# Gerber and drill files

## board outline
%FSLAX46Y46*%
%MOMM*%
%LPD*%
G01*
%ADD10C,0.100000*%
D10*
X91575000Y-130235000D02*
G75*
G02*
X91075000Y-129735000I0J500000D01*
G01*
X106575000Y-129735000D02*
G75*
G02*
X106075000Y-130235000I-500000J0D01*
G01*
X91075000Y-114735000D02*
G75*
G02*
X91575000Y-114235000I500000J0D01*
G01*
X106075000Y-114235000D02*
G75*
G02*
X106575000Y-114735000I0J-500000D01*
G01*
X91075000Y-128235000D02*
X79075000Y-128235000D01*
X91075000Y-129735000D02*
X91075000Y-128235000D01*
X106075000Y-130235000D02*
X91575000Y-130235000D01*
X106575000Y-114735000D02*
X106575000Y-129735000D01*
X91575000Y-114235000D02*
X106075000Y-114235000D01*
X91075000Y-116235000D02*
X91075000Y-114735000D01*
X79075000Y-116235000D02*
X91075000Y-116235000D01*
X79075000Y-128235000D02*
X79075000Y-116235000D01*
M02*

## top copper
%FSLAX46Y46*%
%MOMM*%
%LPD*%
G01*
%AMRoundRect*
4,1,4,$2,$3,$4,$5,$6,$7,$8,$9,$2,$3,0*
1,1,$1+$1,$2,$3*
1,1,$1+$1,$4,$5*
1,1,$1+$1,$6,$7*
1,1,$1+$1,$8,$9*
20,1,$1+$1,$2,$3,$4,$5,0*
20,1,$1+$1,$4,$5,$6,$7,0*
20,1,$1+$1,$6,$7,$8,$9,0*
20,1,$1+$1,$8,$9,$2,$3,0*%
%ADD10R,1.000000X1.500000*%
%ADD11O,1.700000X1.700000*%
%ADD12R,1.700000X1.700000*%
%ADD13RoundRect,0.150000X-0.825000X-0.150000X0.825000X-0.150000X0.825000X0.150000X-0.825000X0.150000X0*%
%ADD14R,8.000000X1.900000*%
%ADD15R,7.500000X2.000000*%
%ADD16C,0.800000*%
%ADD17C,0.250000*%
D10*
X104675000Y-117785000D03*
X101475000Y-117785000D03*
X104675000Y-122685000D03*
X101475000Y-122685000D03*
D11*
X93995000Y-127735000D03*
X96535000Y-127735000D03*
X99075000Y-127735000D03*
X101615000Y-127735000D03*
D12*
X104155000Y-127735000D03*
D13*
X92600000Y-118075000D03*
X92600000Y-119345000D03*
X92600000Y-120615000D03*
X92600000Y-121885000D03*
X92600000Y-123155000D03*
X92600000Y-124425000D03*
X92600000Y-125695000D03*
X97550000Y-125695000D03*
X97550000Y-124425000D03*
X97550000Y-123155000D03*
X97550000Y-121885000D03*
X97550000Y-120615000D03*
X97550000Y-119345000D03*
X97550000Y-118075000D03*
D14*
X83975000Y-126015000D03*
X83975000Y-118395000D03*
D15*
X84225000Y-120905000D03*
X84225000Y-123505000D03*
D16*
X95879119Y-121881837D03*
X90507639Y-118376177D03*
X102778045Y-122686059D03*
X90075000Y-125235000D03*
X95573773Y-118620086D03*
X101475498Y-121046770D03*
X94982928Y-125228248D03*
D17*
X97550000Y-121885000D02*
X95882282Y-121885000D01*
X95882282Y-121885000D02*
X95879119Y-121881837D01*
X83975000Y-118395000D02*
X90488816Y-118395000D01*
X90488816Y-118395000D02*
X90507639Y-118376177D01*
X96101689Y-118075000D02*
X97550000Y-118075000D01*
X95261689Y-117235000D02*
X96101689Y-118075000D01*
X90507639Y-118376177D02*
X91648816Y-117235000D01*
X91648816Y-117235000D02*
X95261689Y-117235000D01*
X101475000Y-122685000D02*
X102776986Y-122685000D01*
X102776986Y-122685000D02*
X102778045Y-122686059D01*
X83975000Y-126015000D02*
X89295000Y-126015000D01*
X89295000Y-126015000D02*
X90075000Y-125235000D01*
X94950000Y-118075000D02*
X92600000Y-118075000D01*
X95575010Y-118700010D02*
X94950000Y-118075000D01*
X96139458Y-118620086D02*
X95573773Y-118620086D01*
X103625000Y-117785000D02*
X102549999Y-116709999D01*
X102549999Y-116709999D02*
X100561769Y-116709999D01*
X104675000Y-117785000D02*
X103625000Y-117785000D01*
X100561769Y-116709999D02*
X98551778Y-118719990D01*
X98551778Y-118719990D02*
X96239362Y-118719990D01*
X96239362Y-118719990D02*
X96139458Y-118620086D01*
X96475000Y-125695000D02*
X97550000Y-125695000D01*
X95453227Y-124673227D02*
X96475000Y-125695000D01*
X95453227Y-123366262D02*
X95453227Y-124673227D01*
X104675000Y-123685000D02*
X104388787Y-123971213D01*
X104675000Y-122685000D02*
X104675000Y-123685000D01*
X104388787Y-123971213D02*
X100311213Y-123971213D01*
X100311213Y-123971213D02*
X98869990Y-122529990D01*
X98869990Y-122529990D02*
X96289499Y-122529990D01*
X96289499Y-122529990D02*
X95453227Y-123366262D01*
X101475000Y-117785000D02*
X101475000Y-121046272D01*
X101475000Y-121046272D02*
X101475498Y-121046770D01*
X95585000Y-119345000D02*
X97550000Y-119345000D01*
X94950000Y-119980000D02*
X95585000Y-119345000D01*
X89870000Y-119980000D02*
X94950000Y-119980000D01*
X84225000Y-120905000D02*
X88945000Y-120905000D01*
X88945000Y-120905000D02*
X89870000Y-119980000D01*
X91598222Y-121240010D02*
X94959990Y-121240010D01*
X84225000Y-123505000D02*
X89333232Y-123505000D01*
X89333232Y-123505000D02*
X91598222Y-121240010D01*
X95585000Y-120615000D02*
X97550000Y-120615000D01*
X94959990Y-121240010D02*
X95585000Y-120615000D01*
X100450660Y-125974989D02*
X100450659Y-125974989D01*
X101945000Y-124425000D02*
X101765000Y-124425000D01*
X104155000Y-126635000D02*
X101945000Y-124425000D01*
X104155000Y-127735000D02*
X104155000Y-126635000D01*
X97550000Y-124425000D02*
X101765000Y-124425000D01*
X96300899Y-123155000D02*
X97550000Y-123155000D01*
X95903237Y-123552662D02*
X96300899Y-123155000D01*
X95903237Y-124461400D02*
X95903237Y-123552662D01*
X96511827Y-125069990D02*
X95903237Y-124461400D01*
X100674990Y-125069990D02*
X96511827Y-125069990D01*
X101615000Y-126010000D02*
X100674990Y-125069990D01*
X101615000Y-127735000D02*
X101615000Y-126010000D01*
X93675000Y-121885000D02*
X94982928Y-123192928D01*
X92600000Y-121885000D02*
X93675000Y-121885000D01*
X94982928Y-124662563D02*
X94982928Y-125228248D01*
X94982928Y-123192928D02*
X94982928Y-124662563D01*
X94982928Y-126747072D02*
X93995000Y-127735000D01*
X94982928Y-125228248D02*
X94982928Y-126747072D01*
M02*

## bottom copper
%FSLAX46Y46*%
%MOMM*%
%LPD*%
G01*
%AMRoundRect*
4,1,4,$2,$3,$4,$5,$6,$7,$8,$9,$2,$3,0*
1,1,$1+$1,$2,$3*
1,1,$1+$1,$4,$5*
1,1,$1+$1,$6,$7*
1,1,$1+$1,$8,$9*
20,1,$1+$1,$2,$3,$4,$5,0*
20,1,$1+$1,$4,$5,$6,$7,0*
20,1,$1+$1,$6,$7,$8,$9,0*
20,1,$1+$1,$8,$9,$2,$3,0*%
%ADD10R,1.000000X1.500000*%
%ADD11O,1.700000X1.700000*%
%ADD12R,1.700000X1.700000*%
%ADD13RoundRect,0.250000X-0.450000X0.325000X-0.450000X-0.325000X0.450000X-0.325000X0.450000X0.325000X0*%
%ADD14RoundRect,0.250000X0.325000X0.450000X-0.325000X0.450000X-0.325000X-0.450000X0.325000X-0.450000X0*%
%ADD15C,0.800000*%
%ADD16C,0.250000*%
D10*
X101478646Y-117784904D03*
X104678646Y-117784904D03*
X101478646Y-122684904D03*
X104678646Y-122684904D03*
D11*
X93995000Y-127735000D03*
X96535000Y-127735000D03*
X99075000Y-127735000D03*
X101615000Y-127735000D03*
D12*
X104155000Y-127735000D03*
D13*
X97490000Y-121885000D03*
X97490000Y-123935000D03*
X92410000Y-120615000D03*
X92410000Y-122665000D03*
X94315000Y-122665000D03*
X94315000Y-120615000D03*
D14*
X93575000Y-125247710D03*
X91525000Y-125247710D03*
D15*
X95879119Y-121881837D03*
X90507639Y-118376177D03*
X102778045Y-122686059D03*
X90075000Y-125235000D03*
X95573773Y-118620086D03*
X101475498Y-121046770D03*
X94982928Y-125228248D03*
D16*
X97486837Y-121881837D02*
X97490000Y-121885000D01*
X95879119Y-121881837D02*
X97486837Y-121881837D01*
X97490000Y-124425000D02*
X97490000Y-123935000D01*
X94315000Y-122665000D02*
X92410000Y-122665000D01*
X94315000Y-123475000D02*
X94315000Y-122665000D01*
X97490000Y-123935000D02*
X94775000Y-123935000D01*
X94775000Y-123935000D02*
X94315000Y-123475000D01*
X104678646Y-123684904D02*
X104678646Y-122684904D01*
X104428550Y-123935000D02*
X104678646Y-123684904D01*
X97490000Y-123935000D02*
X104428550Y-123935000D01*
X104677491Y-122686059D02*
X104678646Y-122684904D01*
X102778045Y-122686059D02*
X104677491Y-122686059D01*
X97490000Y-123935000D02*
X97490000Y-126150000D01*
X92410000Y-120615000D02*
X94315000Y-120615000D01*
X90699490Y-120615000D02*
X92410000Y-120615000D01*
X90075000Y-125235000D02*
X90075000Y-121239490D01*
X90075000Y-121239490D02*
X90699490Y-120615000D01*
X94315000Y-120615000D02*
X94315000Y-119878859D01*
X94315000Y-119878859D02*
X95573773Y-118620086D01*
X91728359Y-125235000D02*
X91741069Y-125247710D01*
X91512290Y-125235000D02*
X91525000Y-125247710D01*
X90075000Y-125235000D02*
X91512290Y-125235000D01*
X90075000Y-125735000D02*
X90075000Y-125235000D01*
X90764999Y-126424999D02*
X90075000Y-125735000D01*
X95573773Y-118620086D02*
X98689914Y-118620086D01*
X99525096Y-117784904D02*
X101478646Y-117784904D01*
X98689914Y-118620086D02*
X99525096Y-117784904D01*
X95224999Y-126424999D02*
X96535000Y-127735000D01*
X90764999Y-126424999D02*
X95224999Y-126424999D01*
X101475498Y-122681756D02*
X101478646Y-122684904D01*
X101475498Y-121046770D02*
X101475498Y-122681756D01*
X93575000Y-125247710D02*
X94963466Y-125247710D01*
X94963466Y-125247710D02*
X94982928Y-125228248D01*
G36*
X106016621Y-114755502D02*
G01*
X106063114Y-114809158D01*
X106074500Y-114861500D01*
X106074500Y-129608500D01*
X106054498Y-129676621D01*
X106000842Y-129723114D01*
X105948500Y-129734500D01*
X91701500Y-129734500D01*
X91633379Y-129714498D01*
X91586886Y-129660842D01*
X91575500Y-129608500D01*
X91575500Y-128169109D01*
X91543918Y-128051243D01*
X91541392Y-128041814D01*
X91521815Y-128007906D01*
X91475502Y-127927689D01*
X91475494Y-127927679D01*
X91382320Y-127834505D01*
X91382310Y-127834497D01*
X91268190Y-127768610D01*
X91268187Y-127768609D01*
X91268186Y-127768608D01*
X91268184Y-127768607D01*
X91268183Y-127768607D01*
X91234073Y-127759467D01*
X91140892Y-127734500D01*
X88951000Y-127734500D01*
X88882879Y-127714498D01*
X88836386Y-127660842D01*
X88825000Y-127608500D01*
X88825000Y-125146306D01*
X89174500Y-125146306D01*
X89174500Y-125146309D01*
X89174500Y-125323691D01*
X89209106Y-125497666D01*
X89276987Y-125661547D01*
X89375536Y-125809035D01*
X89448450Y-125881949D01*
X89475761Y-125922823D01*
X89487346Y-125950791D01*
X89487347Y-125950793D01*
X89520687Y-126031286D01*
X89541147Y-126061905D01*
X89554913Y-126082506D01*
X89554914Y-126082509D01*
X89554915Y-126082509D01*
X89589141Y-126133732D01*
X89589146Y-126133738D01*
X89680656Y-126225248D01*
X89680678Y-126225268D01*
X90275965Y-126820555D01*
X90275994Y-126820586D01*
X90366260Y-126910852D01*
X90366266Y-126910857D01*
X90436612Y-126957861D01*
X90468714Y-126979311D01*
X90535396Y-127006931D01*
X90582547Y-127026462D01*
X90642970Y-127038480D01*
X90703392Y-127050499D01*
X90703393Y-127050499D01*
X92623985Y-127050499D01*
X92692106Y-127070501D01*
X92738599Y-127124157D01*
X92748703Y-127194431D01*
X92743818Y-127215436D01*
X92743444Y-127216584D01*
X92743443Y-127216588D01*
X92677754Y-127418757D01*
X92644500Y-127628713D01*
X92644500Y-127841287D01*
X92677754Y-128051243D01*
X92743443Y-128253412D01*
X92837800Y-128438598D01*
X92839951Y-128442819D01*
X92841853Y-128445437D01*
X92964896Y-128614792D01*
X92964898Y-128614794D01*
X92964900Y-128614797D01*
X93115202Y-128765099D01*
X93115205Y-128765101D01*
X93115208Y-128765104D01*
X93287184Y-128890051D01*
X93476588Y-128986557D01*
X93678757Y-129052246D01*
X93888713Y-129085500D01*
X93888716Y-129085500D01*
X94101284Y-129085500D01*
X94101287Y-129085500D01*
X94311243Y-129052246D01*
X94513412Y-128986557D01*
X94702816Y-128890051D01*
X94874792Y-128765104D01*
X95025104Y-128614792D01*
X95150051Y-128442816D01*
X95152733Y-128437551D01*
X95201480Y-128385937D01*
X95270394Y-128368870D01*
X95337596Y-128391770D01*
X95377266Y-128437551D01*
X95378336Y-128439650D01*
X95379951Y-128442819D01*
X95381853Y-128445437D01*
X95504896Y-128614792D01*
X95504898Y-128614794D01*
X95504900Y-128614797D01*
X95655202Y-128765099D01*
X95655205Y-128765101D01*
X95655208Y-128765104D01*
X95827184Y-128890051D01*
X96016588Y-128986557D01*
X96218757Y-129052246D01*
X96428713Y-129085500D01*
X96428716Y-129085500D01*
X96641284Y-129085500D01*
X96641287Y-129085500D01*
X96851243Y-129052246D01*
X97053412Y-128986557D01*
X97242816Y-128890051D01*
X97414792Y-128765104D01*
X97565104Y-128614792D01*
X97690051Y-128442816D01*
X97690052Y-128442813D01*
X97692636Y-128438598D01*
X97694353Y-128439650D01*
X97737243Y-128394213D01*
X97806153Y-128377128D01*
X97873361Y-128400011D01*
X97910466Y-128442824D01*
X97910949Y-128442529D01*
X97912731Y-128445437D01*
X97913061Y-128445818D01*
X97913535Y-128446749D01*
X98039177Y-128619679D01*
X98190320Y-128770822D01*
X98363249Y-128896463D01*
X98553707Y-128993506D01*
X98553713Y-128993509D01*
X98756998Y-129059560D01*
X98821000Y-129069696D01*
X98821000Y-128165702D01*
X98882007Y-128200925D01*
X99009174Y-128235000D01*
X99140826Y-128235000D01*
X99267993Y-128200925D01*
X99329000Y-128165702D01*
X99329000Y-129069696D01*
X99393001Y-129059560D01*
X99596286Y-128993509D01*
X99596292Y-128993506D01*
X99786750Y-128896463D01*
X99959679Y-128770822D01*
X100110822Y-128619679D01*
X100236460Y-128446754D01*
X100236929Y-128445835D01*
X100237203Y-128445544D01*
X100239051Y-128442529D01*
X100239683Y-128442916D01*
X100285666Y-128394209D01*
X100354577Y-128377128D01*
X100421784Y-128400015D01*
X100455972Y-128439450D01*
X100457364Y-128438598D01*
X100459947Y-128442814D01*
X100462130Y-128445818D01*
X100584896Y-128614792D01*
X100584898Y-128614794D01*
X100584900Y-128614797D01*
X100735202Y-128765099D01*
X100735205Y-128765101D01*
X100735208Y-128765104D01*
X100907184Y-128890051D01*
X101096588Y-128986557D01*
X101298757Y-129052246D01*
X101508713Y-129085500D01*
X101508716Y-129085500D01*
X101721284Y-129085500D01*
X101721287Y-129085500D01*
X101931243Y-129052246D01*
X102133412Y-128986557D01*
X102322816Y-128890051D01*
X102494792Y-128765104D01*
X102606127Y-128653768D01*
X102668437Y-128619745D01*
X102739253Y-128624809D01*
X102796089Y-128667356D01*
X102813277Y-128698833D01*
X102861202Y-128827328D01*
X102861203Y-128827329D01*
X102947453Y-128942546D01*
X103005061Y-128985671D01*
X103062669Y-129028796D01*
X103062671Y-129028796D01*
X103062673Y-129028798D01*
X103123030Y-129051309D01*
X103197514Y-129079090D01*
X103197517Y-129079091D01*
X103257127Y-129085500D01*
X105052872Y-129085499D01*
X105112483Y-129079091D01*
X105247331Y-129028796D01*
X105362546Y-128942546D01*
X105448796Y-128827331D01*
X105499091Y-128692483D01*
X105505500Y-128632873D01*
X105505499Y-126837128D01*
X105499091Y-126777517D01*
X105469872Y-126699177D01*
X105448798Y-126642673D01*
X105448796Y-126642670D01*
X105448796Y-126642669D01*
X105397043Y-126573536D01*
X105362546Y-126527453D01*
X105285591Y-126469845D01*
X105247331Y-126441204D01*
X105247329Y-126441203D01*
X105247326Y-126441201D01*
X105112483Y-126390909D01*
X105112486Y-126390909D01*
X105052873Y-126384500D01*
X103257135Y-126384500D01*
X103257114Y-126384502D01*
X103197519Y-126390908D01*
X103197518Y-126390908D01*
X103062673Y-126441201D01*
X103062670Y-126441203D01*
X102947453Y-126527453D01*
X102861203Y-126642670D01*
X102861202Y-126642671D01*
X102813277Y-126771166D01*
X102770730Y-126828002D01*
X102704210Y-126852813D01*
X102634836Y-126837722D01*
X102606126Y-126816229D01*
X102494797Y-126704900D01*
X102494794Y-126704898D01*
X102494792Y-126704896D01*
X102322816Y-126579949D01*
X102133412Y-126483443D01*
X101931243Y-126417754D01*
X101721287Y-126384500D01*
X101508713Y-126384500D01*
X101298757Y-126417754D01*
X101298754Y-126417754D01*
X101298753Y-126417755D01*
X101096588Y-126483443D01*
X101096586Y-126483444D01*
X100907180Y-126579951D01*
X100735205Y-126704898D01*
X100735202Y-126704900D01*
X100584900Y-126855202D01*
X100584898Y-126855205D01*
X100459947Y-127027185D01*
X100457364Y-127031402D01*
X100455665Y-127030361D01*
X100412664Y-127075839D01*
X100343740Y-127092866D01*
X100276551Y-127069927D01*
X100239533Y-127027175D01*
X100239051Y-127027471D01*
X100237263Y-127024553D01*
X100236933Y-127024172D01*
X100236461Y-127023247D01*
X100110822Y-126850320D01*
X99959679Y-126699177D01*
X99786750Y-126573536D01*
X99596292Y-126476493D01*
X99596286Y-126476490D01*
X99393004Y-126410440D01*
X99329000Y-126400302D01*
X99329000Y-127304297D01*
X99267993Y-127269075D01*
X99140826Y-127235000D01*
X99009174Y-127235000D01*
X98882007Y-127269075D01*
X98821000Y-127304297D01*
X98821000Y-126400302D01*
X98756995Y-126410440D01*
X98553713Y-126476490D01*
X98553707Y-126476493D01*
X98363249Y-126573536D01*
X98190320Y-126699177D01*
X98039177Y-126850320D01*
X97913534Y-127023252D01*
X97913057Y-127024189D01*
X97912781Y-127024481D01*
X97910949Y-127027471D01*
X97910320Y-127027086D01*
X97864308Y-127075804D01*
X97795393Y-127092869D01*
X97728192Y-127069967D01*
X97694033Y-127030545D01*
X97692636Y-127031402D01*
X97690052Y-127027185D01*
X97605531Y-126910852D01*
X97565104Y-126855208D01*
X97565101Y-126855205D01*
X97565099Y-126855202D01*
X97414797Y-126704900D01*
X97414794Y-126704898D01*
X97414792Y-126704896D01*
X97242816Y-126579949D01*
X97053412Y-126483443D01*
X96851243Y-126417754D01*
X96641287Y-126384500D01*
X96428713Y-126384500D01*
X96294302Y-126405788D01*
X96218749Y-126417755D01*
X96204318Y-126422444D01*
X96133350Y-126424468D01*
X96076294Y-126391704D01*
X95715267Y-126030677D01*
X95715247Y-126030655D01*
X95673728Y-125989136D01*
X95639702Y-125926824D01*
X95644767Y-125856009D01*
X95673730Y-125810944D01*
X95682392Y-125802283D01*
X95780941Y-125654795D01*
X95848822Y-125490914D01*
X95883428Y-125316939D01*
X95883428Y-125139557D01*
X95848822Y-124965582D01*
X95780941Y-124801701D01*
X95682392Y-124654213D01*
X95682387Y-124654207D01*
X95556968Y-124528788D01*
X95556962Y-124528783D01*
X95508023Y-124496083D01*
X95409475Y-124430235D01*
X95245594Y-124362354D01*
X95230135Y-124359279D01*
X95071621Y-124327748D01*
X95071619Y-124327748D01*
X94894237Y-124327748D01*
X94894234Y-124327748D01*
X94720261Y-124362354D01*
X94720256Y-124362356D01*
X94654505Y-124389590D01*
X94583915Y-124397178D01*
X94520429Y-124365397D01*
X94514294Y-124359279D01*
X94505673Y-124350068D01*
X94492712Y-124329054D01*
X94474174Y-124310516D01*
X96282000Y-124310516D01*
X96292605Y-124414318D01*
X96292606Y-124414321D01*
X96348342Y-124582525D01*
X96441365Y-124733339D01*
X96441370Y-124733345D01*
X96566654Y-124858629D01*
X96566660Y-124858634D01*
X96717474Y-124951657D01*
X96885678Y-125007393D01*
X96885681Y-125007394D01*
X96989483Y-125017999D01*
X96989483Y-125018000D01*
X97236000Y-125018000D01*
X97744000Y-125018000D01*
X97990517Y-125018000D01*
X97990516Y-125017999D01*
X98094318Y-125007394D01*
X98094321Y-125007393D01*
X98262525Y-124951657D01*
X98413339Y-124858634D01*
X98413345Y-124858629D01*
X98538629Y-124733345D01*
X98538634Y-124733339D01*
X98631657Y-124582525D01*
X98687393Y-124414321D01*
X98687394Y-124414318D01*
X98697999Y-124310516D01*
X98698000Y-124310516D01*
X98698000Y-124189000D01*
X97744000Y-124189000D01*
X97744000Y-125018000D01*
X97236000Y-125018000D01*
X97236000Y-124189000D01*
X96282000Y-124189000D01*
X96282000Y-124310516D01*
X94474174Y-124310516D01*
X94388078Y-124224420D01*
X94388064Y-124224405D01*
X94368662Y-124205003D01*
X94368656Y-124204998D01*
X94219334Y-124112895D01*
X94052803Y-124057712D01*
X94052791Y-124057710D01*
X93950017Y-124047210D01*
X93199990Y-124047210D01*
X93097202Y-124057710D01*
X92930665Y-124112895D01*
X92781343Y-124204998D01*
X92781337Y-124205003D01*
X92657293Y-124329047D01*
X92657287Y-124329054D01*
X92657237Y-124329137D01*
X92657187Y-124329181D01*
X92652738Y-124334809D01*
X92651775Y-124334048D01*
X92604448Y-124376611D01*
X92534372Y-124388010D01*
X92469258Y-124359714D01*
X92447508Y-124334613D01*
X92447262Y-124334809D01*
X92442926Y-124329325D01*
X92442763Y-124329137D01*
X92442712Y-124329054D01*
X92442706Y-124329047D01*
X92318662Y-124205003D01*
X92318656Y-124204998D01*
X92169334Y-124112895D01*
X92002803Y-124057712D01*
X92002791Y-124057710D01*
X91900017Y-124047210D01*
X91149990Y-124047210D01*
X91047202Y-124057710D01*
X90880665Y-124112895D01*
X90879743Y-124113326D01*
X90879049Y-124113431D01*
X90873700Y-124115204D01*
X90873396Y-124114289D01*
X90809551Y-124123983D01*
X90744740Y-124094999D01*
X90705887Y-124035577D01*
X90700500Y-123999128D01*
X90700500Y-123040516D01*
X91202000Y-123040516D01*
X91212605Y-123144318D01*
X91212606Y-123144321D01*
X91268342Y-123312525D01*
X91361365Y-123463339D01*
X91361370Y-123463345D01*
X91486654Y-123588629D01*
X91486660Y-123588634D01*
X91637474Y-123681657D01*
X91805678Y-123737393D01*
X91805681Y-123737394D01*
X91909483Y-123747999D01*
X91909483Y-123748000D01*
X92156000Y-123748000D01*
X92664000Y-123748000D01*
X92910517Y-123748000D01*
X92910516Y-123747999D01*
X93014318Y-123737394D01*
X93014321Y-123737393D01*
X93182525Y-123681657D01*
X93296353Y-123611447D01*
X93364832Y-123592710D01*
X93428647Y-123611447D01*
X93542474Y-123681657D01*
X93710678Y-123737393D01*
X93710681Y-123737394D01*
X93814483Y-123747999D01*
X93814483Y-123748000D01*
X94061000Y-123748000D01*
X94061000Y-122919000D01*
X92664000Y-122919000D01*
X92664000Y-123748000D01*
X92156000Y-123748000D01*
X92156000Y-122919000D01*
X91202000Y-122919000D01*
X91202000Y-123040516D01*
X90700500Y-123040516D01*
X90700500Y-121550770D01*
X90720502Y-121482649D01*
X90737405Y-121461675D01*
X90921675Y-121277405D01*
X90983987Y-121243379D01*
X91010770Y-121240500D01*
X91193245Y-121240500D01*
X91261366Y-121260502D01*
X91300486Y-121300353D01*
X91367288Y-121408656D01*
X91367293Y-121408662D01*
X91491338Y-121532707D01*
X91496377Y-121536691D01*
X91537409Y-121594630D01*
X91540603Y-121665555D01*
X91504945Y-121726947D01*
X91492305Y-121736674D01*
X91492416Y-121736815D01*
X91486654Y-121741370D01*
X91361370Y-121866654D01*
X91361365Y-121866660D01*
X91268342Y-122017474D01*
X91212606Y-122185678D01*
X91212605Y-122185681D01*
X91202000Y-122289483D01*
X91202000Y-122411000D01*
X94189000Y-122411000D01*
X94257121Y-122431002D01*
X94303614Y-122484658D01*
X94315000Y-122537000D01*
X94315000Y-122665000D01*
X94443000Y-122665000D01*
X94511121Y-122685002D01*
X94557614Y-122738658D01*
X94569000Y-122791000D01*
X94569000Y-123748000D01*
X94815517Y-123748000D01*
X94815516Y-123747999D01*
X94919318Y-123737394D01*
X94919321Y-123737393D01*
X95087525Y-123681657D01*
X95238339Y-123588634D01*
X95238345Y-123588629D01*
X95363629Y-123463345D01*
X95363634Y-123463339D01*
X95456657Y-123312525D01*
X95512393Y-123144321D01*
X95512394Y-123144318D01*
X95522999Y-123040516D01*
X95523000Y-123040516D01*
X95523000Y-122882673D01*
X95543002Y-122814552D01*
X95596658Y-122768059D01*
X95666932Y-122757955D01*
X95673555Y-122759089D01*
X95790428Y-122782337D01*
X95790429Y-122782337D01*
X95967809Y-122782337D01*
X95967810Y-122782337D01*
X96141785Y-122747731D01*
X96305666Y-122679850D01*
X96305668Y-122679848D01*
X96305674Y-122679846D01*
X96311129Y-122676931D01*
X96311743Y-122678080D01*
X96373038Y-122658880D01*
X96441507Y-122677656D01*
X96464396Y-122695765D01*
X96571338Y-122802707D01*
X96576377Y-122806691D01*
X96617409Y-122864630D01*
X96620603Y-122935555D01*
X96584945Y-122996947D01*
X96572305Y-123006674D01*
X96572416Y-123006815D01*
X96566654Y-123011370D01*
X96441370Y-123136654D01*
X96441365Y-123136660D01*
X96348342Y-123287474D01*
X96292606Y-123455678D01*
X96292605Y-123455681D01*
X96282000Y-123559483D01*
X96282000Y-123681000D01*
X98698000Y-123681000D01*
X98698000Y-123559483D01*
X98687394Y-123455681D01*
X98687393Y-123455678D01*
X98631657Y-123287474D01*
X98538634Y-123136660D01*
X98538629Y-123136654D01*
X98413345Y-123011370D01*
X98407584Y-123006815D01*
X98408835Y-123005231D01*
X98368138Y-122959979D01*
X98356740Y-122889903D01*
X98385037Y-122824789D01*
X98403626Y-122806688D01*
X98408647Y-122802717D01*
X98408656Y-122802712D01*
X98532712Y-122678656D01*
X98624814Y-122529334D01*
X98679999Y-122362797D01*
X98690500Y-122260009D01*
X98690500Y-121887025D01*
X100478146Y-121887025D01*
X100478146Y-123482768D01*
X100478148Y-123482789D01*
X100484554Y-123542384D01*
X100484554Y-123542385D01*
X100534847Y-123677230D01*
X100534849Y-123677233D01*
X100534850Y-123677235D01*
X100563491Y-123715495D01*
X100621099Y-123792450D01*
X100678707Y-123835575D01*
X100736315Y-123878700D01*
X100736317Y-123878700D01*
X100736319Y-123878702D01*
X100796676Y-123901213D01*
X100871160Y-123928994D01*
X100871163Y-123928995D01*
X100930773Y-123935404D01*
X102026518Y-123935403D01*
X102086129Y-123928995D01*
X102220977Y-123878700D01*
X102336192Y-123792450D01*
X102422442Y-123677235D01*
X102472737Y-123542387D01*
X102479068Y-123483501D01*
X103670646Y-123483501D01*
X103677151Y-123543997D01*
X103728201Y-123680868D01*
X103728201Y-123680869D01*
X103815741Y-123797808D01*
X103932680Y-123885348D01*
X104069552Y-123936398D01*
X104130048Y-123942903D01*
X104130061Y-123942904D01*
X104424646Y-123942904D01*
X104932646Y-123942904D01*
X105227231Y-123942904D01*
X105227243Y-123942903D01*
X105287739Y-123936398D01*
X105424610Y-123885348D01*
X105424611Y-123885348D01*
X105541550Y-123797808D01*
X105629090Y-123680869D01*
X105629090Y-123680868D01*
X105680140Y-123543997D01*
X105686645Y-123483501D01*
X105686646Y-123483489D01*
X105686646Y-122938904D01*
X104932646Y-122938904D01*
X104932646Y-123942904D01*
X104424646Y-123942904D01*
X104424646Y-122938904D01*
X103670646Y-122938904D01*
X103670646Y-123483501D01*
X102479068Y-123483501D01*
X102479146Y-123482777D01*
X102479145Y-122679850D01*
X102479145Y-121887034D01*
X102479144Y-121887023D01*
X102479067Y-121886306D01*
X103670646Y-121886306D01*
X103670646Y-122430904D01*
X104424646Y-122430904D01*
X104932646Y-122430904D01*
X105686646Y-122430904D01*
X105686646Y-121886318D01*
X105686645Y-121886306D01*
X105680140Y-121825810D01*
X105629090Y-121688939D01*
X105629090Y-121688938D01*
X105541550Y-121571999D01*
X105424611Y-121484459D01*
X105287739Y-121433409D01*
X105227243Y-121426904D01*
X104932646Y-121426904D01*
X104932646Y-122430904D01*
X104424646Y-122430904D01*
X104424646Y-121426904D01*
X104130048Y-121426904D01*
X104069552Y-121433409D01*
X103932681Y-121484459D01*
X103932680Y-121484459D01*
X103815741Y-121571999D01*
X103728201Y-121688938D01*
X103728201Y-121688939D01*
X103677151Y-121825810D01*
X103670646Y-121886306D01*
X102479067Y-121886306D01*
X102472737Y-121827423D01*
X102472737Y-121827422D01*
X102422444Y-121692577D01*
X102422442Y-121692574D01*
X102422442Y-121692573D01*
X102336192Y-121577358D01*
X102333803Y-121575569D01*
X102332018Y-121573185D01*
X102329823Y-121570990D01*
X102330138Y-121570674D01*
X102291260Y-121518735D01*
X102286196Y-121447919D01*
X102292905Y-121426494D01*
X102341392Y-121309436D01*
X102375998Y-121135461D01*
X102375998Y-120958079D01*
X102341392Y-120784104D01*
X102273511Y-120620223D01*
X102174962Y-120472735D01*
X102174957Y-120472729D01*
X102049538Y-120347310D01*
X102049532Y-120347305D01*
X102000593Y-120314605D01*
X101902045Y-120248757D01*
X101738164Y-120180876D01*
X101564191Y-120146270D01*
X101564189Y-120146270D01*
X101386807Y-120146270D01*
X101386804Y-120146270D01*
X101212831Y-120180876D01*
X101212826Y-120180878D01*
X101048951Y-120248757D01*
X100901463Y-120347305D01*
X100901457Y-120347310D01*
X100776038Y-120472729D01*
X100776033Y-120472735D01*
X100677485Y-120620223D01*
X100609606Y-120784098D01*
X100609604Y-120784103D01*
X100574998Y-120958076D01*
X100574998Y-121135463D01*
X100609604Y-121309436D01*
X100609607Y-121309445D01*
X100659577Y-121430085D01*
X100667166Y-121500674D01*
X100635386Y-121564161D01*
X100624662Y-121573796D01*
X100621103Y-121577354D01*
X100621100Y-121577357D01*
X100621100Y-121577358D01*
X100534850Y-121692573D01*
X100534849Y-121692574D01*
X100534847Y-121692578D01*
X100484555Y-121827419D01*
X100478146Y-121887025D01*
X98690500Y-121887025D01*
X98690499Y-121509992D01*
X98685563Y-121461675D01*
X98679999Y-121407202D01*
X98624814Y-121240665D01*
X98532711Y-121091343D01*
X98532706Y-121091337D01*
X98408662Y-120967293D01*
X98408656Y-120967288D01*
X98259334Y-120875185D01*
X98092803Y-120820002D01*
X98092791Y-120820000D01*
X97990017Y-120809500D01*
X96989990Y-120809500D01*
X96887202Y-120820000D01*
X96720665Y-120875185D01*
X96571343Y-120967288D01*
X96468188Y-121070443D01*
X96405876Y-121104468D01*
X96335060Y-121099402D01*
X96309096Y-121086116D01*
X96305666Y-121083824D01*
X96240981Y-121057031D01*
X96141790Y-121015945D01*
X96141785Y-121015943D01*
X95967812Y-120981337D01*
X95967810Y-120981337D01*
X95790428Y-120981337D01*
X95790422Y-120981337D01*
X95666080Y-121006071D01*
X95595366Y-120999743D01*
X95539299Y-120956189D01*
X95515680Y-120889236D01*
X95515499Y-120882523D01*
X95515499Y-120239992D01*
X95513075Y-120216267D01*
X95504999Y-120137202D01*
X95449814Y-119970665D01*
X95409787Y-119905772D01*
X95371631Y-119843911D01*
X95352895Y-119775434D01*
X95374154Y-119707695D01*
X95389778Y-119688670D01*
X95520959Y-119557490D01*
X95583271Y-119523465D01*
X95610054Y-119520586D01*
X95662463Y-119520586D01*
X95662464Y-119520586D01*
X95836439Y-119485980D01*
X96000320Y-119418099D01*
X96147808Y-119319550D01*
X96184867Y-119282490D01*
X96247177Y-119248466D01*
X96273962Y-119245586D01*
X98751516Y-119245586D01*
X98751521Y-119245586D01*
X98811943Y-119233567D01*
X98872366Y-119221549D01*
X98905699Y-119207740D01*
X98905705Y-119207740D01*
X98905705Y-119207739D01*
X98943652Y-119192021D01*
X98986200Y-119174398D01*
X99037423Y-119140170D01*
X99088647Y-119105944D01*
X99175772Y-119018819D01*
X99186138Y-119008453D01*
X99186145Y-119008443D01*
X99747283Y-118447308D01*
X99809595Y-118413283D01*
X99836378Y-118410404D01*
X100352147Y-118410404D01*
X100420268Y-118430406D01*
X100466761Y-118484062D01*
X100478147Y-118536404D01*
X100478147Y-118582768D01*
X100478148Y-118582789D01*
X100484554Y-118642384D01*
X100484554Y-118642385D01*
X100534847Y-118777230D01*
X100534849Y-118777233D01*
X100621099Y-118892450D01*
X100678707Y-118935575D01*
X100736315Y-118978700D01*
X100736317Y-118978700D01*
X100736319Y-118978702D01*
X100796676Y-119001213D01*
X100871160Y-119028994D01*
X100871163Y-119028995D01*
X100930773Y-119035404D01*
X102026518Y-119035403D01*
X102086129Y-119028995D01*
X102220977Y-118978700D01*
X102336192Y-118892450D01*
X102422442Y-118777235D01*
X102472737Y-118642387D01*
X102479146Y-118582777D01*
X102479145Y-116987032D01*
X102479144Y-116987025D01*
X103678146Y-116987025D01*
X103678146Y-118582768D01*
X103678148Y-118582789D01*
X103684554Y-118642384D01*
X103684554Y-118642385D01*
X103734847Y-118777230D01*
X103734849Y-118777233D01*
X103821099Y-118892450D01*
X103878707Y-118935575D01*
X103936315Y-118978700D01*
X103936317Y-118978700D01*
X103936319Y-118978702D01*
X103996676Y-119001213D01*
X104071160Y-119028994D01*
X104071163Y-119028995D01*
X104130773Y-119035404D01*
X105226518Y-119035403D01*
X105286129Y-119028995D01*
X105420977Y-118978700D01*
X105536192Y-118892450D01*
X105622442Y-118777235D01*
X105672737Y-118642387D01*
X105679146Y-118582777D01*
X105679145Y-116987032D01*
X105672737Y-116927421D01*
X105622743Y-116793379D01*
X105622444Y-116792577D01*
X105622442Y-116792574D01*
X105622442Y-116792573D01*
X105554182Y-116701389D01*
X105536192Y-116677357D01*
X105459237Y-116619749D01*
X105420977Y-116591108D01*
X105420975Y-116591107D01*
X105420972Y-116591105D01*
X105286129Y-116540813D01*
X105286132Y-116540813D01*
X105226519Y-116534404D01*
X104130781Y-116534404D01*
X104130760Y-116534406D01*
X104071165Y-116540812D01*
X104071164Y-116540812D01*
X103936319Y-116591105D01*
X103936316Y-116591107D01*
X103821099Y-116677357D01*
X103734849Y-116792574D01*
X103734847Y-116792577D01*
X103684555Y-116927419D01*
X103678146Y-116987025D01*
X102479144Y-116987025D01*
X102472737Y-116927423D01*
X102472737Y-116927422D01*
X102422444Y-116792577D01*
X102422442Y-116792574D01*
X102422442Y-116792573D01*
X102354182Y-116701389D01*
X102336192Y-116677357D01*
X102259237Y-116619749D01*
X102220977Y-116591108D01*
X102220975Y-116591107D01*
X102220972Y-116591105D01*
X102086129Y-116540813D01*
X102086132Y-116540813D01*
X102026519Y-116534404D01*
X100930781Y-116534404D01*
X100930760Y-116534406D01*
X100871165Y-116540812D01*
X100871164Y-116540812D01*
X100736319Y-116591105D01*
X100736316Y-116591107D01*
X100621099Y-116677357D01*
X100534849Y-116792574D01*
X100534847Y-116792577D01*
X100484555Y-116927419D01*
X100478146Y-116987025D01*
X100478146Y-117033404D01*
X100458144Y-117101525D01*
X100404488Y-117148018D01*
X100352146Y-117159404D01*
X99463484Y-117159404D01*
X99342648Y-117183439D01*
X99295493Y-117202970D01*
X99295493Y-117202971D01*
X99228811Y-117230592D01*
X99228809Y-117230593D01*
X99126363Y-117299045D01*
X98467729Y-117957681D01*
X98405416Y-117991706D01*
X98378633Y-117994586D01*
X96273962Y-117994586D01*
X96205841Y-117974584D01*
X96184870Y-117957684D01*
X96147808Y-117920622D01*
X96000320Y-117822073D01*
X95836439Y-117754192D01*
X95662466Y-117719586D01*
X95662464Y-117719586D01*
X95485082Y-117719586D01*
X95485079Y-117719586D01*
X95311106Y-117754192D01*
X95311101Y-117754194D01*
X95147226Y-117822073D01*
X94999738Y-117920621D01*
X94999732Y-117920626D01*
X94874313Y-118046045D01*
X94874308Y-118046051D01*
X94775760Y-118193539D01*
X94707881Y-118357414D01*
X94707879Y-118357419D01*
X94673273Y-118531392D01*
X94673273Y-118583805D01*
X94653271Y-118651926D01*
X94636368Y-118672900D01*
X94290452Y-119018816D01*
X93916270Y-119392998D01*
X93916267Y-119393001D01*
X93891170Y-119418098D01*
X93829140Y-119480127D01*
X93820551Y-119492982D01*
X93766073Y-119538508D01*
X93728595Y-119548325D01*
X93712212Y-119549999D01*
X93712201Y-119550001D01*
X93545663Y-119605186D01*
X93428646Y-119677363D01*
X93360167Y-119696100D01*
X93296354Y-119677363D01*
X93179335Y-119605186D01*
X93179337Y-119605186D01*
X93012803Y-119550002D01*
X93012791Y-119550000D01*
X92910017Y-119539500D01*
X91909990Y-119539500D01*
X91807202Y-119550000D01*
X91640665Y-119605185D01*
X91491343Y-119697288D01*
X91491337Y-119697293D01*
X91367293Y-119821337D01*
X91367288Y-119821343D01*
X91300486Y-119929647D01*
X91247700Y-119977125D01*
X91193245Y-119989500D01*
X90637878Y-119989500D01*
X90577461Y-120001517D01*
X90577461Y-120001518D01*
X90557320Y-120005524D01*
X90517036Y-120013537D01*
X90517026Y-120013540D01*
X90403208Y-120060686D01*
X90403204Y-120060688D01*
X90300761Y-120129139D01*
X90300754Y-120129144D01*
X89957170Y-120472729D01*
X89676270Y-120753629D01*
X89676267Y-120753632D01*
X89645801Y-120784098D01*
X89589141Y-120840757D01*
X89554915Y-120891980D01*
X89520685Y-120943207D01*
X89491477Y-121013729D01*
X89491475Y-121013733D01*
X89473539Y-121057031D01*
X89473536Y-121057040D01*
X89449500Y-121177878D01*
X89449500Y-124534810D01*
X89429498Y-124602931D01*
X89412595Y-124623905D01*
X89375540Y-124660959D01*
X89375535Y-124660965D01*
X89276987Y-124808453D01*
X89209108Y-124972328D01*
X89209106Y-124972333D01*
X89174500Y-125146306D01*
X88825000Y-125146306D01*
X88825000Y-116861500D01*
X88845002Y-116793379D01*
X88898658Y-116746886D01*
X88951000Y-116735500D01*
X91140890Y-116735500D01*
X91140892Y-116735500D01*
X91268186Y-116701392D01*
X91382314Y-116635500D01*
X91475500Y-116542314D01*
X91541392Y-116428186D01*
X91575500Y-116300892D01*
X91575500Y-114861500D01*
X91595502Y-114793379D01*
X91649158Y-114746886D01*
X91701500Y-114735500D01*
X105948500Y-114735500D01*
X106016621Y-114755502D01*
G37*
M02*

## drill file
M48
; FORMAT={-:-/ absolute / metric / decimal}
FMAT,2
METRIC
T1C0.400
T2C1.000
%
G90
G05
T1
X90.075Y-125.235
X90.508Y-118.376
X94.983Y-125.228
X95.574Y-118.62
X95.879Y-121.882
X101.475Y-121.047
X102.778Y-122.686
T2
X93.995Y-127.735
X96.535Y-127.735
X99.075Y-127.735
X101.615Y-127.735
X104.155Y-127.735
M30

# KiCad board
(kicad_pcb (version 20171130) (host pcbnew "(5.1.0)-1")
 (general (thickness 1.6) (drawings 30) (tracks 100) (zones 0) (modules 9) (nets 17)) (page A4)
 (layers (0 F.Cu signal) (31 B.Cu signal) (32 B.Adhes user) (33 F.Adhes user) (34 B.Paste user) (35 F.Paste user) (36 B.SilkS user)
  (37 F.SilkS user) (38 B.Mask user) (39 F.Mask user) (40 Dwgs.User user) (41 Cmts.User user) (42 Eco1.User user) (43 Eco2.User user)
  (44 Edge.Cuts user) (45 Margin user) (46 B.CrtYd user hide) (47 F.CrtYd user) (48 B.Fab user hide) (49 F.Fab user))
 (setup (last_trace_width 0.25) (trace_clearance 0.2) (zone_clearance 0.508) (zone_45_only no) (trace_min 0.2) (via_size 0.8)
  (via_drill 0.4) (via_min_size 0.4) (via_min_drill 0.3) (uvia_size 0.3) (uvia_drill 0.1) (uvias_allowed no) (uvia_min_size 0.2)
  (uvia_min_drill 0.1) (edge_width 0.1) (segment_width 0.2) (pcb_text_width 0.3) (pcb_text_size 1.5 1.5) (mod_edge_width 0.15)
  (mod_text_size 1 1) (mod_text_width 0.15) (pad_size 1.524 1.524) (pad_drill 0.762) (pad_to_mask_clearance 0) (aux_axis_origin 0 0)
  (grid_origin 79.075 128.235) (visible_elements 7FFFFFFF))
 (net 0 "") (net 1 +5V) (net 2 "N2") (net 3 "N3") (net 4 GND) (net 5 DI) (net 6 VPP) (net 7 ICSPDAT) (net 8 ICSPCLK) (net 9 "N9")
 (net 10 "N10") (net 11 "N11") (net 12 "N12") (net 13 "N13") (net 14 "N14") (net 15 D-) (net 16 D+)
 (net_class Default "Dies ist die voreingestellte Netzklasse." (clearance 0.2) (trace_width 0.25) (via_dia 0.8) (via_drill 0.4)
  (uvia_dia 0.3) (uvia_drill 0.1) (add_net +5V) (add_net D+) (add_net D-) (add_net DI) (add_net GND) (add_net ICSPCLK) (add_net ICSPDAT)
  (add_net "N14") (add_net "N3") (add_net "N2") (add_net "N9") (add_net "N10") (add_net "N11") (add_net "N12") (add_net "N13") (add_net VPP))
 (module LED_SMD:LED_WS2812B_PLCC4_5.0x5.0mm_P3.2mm (layer B.Cu) (at 103.078646 120.234904 270)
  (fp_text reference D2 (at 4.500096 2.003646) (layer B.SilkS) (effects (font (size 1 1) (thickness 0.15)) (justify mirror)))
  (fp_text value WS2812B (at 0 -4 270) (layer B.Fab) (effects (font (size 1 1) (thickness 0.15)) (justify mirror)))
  (pad 1 smd rect (at -2.45 1.6 270) (size 1.5 1) (layers B.Cu B.Paste B.Mask) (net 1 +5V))
  (pad 2 smd rect (at -2.45 -1.6 270) (size 1.5 1) (layers B.Cu B.Paste B.Mask) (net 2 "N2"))
  (pad 4 smd rect (at 2.45 1.6 270) (size 1.5 1) (layers B.Cu B.Paste B.Mask) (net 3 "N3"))
  (pad 3 smd rect (at 2.45 -1.6 270) (size 1.5 1) (layers B.Cu B.Paste B.Mask) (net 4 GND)))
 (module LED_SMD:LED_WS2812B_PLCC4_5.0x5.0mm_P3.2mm (layer F.Cu) (at 103.075 120.235 270)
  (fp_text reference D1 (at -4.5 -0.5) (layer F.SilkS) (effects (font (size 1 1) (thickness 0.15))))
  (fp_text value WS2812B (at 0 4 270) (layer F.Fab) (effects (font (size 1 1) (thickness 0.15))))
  (pad 1 smd rect (at -2.45 -1.6 270) (size 1.5 1) (layers F.Cu F.Paste F.Mask) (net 1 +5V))
  (pad 2 smd rect (at -2.45 1.6 270) (size 1.5 1) (layers F.Cu F.Paste F.Mask) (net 3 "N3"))
  (pad 4 smd rect (at 2.45 -1.6 270) (size 1.5 1) (layers F.Cu F.Paste F.Mask) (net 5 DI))
  (pad 3 smd rect (at 2.45 1.6 270) (size 1.5 1) (layers F.Cu F.Paste F.Mask) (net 4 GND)))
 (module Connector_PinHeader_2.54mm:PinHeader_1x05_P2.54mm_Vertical (layer F.Cu) (at 104.155 127.735 270)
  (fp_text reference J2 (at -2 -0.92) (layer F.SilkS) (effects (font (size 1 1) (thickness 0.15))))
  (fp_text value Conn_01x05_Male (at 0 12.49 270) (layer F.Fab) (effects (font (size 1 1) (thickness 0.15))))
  (pad 5 thru_hole oval (at 0 10.16 270) (size 1.7 1.7) (drill 1) (layers *.Cu *.Mask) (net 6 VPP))
  (pad 4 thru_hole oval (at 0 7.62 270) (size 1.7 1.7) (drill 1) (layers *.Cu *.Mask) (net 1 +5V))
  (pad 3 thru_hole oval (at 0 5.08 270) (size 1.7 1.7) (drill 1) (layers *.Cu *.Mask) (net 4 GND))
  (pad 2 thru_hole oval (at 0 2.54 270) (size 1.7 1.7) (drill 1) (layers *.Cu *.Mask) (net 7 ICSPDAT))
  (pad 1 thru_hole rect (at 0 0 270) (size 1.7 1.7) (drill 1) (layers *.Cu *.Mask) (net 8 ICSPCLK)))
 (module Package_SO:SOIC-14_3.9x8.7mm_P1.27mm (layer F.Cu) (at 95.075 121.885)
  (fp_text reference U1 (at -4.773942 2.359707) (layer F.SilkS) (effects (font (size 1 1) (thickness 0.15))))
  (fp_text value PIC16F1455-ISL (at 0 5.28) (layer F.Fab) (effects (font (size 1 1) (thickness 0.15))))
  (pad 1 smd roundrect (at -2.475 -3.81) (size 1.95 0.6) (layers F.Cu F.Paste F.Mask) (roundrect_rratio 0.25) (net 1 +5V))
  (pad 2 smd roundrect (at -2.475 -2.54) (size 1.95 0.6) (layers F.Cu F.Paste F.Mask) (roundrect_rratio 0.25) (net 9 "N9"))
  (pad 3 smd roundrect (at -2.475 -1.27) (size 1.95 0.6) (layers F.Cu F.Paste F.Mask) (roundrect_rratio 0.25) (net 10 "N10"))
  (pad 4 smd roundrect (at -2.475 0) (size 1.95 0.6) (layers F.Cu F.Paste F.Mask) (roundrect_rratio 0.25) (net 6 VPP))
  (pad 5 smd roundrect (at -2.475 1.27) (size 1.95 0.6) (layers F.Cu F.Paste F.Mask) (roundrect_rratio 0.25) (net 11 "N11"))
  (pad 6 smd roundrect (at -2.475 2.54) (size 1.95 0.6) (layers F.Cu F.Paste F.Mask) (roundrect_rratio 0.25) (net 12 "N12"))
  (pad 7 smd roundrect (at -2.475 3.81) (size 1.95 0.6) (layers F.Cu F.Paste F.Mask) (roundrect_rratio 0.25) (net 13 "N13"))
  (pad 8 smd roundrect (at 2.475 3.81) (size 1.95 0.6) (layers F.Cu F.Paste F.Mask) (roundrect_rratio 0.25) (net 5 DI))
  (pad 9 smd roundrect (at 2.475 2.54) (size 1.95 0.6) (layers F.Cu F.Paste F.Mask) (roundrect_rratio 0.25) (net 8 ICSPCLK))
  (pad 10 smd roundrect (at 2.475 1.27) (size 1.95 0.6) (layers F.Cu F.Paste F.Mask) (roundrect_rratio 0.25) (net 7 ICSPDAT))
  (pad 11 smd roundrect (at 2.475 0) (size 1.95 0.6) (layers F.Cu F.Paste F.Mask) (roundrect_rratio 0.25) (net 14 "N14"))
  (pad 12 smd roundrect (at 2.475 -1.27) (size 1.95 0.6) (layers F.Cu F.Paste F.Mask) (roundrect_rratio 0.25) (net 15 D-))
  (pad 13 smd roundrect (at 2.475 -2.54) (size 1.95 0.6) (layers F.Cu F.Paste F.Mask) (roundrect_rratio 0.25) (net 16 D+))
  (pad 14 smd roundrect (at 2.475 -3.81) (size 1.95 0.6) (layers F.Cu F.Paste F.Mask) (roundrect_rratio 0.25) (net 4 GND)))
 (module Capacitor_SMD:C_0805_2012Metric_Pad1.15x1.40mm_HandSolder (layer B.Cu) (at 97.49 122.91 270)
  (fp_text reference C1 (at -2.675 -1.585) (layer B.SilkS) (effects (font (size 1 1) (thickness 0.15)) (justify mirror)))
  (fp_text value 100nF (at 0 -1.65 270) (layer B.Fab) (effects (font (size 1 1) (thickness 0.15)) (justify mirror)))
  (pad 1 smd roundrect (at -1.025 0 270) (size 1.15 1.4) (layers B.Cu B.Paste B.Mask) (roundrect_rratio 0.217391) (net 14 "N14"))
  (pad 2 smd roundrect (at 1.025 0 270) (size 1.15 1.4) (layers B.Cu B.Paste B.Mask) (roundrect_rratio 0.217391) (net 4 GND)))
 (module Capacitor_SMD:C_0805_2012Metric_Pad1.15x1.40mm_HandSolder (layer B.Cu) (at 92.41 121.64 270)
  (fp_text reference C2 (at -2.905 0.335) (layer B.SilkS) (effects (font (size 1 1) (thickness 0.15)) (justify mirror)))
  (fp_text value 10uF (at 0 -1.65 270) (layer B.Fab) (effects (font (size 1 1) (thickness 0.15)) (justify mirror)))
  (pad 1 smd roundrect (at -1.025 0 270) (size 1.15 1.4) (layers B.Cu B.Paste B.Mask) (roundrect_rratio 0.217391) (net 1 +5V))
  (pad 2 smd roundrect (at 1.025 0 270) (size 1.15 1.4) (layers B.Cu B.Paste B.Mask) (roundrect_rratio 0.217391) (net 4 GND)))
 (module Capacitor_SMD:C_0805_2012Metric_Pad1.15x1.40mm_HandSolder (layer B.Cu) (at 94.315 121.64 270)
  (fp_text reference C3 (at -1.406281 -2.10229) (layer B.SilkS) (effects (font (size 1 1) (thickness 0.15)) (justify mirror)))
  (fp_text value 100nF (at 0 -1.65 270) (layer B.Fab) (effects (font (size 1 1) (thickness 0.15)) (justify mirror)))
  (pad 2 smd roundrect (at 1.025 0 270) (size 1.15 1.4) (layers B.Cu B.Paste B.Mask) (roundrect_rratio 0.217391) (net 4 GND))
  (pad 1 smd roundrect (at -1.025 0 270) (size 1.15 1.4) (layers B.Cu B.Paste B.Mask) (roundrect_rratio 0.217391) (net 1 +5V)))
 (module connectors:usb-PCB (layer F.Cu) (at 79.075 122.205 270)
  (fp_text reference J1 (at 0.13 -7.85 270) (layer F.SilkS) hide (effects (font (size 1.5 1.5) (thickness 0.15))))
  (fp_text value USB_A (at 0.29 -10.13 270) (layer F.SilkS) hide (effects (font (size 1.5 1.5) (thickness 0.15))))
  (pad 1 connect rect (at 3.81 -4.9 270) (size 1.9 8) (layers F.Cu F.Mask) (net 1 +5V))
  (pad 4 connect rect (at -3.81 -4.9 270) (size 1.9 8) (layers F.Cu F.Mask) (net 4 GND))
  (pad 3 connect rect (at -1.3 -5.15 270) (size 2 7.5) (layers F.Cu F.Mask) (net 16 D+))
  (pad 2 connect rect (at 1.3 -5.15 270) (size 2 7.5) (layers F.Cu F.Mask) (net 15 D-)))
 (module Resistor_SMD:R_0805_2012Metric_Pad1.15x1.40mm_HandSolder (layer B.Cu) (at 92.55 125.24771 180)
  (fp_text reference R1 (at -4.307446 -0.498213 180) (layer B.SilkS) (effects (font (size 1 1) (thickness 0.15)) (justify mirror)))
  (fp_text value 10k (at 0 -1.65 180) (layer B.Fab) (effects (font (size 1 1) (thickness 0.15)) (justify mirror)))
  (pad 1 smd roundrect (at -1.025 0 180) (size 1.15 1.4) (layers B.Cu B.Paste B.Mask) (roundrect_rratio 0.217391) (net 6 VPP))
  (pad 2 smd roundrect (at 1.025 0 180) (size 1.15 1.4) (layers B.Cu B.Paste B.Mask) (roundrect_rratio 0.217391) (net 1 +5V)))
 (gr_arc (start 91.575 129.735) (end 91.075 129.735) (angle -90) (layer Edge.Cuts) (width 0.1))
 (gr_arc (start 106.075 129.735) (end 106.075 130.235) (angle -90) (layer Edge.Cuts) (width 0.1))
 (gr_arc (start 91.575 114.735) (end 91.575 114.235) (angle -90) (layer Edge.Cuts) (width 0.1))
 (gr_arc (start 106.075 114.735) (end 106.575 114.735) (angle -90) (layer Edge.Cuts) (width 0.1))
 (gr_line (start 91.075 128.235) (end 79.075 128.235) (layer Edge.Cuts) (width 0.1))
 (gr_line (start 91.075 129.735) (end 91.075 128.235) (layer Edge.Cuts) (width 0.1))
 (gr_line (start 106.075 130.235) (end 91.575 130.235) (layer Edge.Cuts) (width 0.1))
 (gr_line (start 106.575 114.735) (end 106.575 129.735) (layer Edge.Cuts) (width 0.1))
 (gr_line (start 91.575 114.235) (end 106.075 114.235) (layer Edge.Cuts) (width 0.1))
 (gr_line (start 91.075 116.235) (end 91.075 114.735) (layer Edge.Cuts) (width 0.1))
 (gr_line (start 79.075 116.235) (end 91.075 116.235) (layer Edge.Cuts) (width 0.1))
 (gr_line (start 79.075 128.235) (end 79.075 116.235) (layer Edge.Cuts) (width 0.1))
 (via (at 95.879119 121.881837) (size 0.8) (drill 0.4) (layers F.Cu B.Cu) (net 14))
 (segment (start 97.55 121.885) (end 95.882282 121.885) (width 0.25) (layer F.Cu) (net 14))
 (segment (start 95.882282 121.885) (end 95.879119 121.881837) (width 0.25) (layer F.Cu) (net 14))
 (segment (start 97.486837 121.881837) (end 97.49 121.885) (width 0.25) (layer B.Cu) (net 14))
 (segment (start 95.879119 121.881837) (end 97.486837 121.881837) (width 0.25) (layer B.Cu) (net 14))
 (segment (start 97.49 124.425) (end 97.49 123.935) (width 0.25) (layer B.Cu) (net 4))
 (segment (start 94.315 122.665) (end 92.41 122.665) (width 0.25) (layer B.Cu) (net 4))
 (segment (start 94.315 123.475) (end 94.315 122.665) (width 0.25) (layer B.Cu) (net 4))
 (segment (start 97.49 123.935) (end 94.775 123.935) (width 0.25) (layer B.Cu) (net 4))
 (segment (start 94.775 123.935) (end 94.315 123.475) (width 0.25) (layer B.Cu) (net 4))
 (via (at 90.507639 118.376177) (size 0.8) (drill 0.4) (layers F.Cu B.Cu) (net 4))
 (segment (start 83.975 118.395) (end 90.488816 118.395) (width 0.25) (layer F.Cu) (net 4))
 (segment (start 90.488816 118.395) (end 90.507639 118.376177) (width 0.25) (layer F.Cu) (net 4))
 (segment (start 96.101689 118.075) (end 97.55 118.075) (width 0.25) (layer F.Cu) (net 4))
 (segment (start 95.261689 117.235) (end 96.101689 118.075) (width 0.25) (layer F.Cu) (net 4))
 (segment (start 90.507639 118.376177) (end 91.648816 117.235) (width 0.25) (layer F.Cu) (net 4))
 (segment (start 91.648816 117.235) (end 95.261689 117.235) (width 0.25) (layer F.Cu) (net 4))
 (segment (start 104.678646 123.684904) (end 104.678646 122.684904) (width 0.25) (layer B.Cu) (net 4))
 (segment (start 104.42855 123.935) (end 104.678646 123.684904) (width 0.25) (layer B.Cu) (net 4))
 (segment (start 97.49 123.935) (end 104.42855 123.935) (width 0.25) (layer B.Cu) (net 4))
 (via (at 102.778045 122.686059) (size 0.8) (drill 0.4) (layers F.Cu B.Cu) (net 4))
 (segment (start 101.475 122.685) (end 102.776986 122.685) (width 0.25) (layer F.Cu) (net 4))
 (segment (start 102.776986 122.685) (end 102.778045 122.686059) (width 0.25) (layer F.Cu) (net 4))
 (segment (start 104.677491 122.686059) (end 104.678646 122.684904) (width 0.25) (layer B.Cu) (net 4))
 (segment (start 102.778045 122.686059) (end 104.677491 122.686059) (width 0.25) (layer B.Cu) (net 4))
 (segment (start 97.49 123.935) (end 97.49 126.15) (width 0.25) (layer B.Cu) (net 4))
 (segment (start 92.41 120.615) (end 94.315 120.615) (width 0.25) (layer B.Cu) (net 1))
 (segment (start 83.975 126.015) (end 89.295 126.015) (width 0.25) (layer F.Cu) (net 1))
 (via (at 90.075 125.235) (size 0.8) (drill 0.4) (layers F.Cu B.Cu) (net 1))
 (segment (start 89.295 126.015) (end 90.075 125.235) (width 0.25) (layer F.Cu) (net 1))
 (segment (start 90.69949 120.615) (end 92.41 120.615) (width 0.25) (layer B.Cu) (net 1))
 (segment (start 90.075 125.235) (end 90.075 121.23949) (width 0.25) (layer B.Cu) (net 1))
 (segment (start 90.075 121.23949) (end 90.69949 120.615) (width 0.25) (layer B.Cu) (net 1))
 (via (at 95.573773 118.620086) (size 0.8) (drill 0.4) (layers F.Cu B.Cu) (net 1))
 (segment (start 94.315 120.615) (end 94.315 119.878859) (width 0.25) (layer B.Cu) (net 1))
 (segment (start 94.315 119.878859) (end 95.573773 118.620086) (width 0.25) (layer B.Cu) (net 1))
 (segment (start 91.728359 125.235) (end 91.741069 125.24771) (width 0.25) (layer B.Cu) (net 1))
 (segment (start 91.51229 125.235) (end 91.525 125.24771) (width 0.25) (layer B.Cu) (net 1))
 (segment (start 90.075 125.235) (end 91.51229 125.235) (width 0.25) (layer B.Cu) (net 1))
 (segment (start 90.075 125.735) (end 90.075 125.235) (width 0.25) (layer B.Cu) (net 1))
 (segment (start 90.764999 126.424999) (end 90.075 125.735) (width 0.25) (layer B.Cu) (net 1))
 (segment (start 94.95 118.075) (end 92.6 118.075) (width 0.25) (layer F.Cu) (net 1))
 (segment (start 95.57501 118.70001) (end 94.95 118.075) (width 0.25) (layer F.Cu) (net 1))
 (segment (start 95.573773 118.620086) (end 98.689914 118.620086) (width 0.25) (layer B.Cu) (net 1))
 (segment (start 99.525096 117.784904) (end 101.478646 117.784904) (width 0.25) (layer B.Cu) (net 1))
 (segment (start 98.689914 118.620086) (end 99.525096 117.784904) (width 0.25) (layer B.Cu) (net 1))
 (segment (start 95.224999 126.424999) (end 96.535 127.735) (width 0.25) (layer B.Cu) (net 1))
 (segment (start 90.764999 126.424999) (end 95.224999 126.424999) (width 0.25) (layer B.Cu) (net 1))
 (segment (start 96.139458 118.620086) (end 95.573773 118.620086) (width 0.25) (layer F.Cu) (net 1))
 (segment (start 103.625 117.785) (end 102.549999 116.709999) (width 0.25) (layer F.Cu) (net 1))
 (segment (start 102.549999 116.709999) (end 100.561769 116.709999) (width 0.25) (layer F.Cu) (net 1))
 (segment (start 104.675 117.785) (end 103.625 117.785) (width 0.25) (layer F.Cu) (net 1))
 (segment (start 100.561769 116.709999) (end 98.551778 118.71999) (width 0.25) (layer F.Cu) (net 1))
 (segment (start 98.551778 118.71999) (end 96.239362 118.71999) (width 0.25) (layer F.Cu) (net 1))
 (segment (start 96.239362 118.71999) (end 96.139458 118.620086) (width 0.25) (layer F.Cu) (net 1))
 (segment (start 96.475 125.695) (end 97.55 125.695) (width 0.25) (layer F.Cu) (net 5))
 (segment (start 95.453227 124.673227) (end 96.475 125.695) (width 0.25) (layer F.Cu) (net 5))
 (segment (start 95.453227 123.366262) (end 95.453227 124.673227) (width 0.25) (layer F.Cu) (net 5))
 (segment (start 104.675 123.685) (end 104.388787 123.971213) (width 0.25) (layer F.Cu) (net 5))
 (segment (start 104.675 122.685) (end 104.675 123.685) (width 0.25) (layer F.Cu) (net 5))
 (segment (start 104.388787 123.971213) (end 100.311213 123.971213) (width 0.25) (layer F.Cu) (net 5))
 (segment (start 100.311213 123.971213) (end 98.86999 122.52999) (width 0.25) (layer F.Cu) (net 5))
 (segment (start 98.86999 122.52999) (end 96.289499 122.52999) (width 0.25) (layer F.Cu) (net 5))
 (segment (start 96.289499 122.52999) (end 95.453227 123.366262) (width 0.25) (layer F.Cu) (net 5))
 (via (at 101.475498 121.04677) (size 0.8) (drill 0.4) (layers F.Cu B.Cu) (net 3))
 (segment (start 101.475 117.785) (end 101.475 121.046272) (width 0.25) (layer F.Cu) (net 3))
 (segment (start 101.475 121.046272) (end 101.475498 121.04677) (width 0.25) (layer F.Cu) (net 3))
 (segment (start 101.475498 122.681756) (end 101.478646 122.684904) (width 0.25) (layer B.Cu) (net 3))
 (segment (start 101.475498 121.04677) (end 101.475498 122.681756) (width 0.25) (layer B.Cu) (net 3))
 (segment (start 95.585 119.345) (end 97.55 119.345) (width 0.25) (layer F.Cu) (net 16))
 (segment (start 94.95 119.98) (end 95.585 119.345) (width 0.25) (layer F.Cu) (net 16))
 (segment (start 89.87 119.98) (end 94.95 119.98) (width 0.25) (layer F.Cu) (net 16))
 (segment (start 84.225 120.905) (end 88.945 120.905) (width 0.25) (layer F.Cu) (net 16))
 (segment (start 88.945 120.905) (end 89.87 119.98) (width 0.25) (layer F.Cu) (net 16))
 (segment (start 91.598222 121.24001) (end 94.95999 121.24001) (width 0.25) (layer F.Cu) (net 15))
 (segment (start 84.225 123.505) (end 89.333232 123.505) (width 0.25) (layer F.Cu) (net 15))
 (segment (start 89.333232 123.505) (end 91.598222 121.24001) (width 0.25) (layer F.Cu) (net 15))
 (segment (start 95.585 120.615) (end 97.55 120.615) (width 0.25) (layer F.Cu) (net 15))
 (segment (start 94.95999 121.24001) (end 95.585 120.615) (width 0.25) (layer F.Cu) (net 15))
 (segment (start 100.45066 125.974989) (end 100.450659 125.974989) (width 0.25) (layer F.Cu) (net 8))
 (segment (start 101.945 124.425) (end 101.765 124.425) (width 0.25) (layer F.Cu) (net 8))
 (segment (start 104.155 126.635) (end 101.945 124.425) (width 0.25) (layer F.Cu) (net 8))
 (segment (start 104.155 127.735) (end 104.155 126.635) (width 0.25) (layer F.Cu) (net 8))
 (segment (start 97.55 124.425) (end 101.765 124.425) (width 0.25) (layer F.Cu) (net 8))
 (segment (start 96.300899 123.155) (end 97.55 123.155) (width 0.25) (layer F.Cu) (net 7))
 (segment (start 95.903237 123.552662) (end 96.300899 123.155) (width 0.25) (layer F.Cu) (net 7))
 (segment (start 95.903237 124.4614) (end 95.903237 123.552662) (width 0.25) (layer F.Cu) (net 7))
 (segment (start 96.511827 125.06999) (end 95.903237 124.4614) (width 0.25) (layer F.Cu) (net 7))
 (segment (start 100.67499 125.06999) (end 96.511827 125.06999) (width 0.25) (layer F.Cu) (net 7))
 (segment (start 101.615 126.01) (end 100.67499 125.06999) (width 0.25) (layer F.Cu) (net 7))
 (segment (start 101.615 127.735) (end 101.615 126.01) (width 0.25) (layer F.Cu) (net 7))
 (segment (start 93.575 125.24771) (end 94.963466 125.24771) (width 0.25) (layer B.Cu) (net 6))
 (segment (start 94.963466 125.24771) (end 94.982928 125.228248) (width 0.25) (layer B.Cu) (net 6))
 (segment (start 93.675 121.885) (end 94.982928 123.192928) (width 0.25) (layer F.Cu) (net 6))
 (segment (start 92.6 121.885) (end 93.675 121.885) (width 0.25) (layer F.Cu) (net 6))
 (segment (start 94.982928 124.662563) (end 94.982928 125.228248) (width 0.25) (layer F.Cu) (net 6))
 (segment (start 94.982928 123.192928) (end 94.982928 124.662563) (width 0.25) (layer F.Cu) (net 6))
 (via (at 94.982928 125.228248) (size 0.8) (drill 0.4) (layers F.Cu B.Cu) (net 6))
 (segment (start 94.982928 126.747072) (end 93.995 127.735) (width 0.25) (layer F.Cu) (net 6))
 (segment (start 94.982928 125.228248) (end 94.982928 126.747072) (width 0.25) (layer F.Cu) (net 6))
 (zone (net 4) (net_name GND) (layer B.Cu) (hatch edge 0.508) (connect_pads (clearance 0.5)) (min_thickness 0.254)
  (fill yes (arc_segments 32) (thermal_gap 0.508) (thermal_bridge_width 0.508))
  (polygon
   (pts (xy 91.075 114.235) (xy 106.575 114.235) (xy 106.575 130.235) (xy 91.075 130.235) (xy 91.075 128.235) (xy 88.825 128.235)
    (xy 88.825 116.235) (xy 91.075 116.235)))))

